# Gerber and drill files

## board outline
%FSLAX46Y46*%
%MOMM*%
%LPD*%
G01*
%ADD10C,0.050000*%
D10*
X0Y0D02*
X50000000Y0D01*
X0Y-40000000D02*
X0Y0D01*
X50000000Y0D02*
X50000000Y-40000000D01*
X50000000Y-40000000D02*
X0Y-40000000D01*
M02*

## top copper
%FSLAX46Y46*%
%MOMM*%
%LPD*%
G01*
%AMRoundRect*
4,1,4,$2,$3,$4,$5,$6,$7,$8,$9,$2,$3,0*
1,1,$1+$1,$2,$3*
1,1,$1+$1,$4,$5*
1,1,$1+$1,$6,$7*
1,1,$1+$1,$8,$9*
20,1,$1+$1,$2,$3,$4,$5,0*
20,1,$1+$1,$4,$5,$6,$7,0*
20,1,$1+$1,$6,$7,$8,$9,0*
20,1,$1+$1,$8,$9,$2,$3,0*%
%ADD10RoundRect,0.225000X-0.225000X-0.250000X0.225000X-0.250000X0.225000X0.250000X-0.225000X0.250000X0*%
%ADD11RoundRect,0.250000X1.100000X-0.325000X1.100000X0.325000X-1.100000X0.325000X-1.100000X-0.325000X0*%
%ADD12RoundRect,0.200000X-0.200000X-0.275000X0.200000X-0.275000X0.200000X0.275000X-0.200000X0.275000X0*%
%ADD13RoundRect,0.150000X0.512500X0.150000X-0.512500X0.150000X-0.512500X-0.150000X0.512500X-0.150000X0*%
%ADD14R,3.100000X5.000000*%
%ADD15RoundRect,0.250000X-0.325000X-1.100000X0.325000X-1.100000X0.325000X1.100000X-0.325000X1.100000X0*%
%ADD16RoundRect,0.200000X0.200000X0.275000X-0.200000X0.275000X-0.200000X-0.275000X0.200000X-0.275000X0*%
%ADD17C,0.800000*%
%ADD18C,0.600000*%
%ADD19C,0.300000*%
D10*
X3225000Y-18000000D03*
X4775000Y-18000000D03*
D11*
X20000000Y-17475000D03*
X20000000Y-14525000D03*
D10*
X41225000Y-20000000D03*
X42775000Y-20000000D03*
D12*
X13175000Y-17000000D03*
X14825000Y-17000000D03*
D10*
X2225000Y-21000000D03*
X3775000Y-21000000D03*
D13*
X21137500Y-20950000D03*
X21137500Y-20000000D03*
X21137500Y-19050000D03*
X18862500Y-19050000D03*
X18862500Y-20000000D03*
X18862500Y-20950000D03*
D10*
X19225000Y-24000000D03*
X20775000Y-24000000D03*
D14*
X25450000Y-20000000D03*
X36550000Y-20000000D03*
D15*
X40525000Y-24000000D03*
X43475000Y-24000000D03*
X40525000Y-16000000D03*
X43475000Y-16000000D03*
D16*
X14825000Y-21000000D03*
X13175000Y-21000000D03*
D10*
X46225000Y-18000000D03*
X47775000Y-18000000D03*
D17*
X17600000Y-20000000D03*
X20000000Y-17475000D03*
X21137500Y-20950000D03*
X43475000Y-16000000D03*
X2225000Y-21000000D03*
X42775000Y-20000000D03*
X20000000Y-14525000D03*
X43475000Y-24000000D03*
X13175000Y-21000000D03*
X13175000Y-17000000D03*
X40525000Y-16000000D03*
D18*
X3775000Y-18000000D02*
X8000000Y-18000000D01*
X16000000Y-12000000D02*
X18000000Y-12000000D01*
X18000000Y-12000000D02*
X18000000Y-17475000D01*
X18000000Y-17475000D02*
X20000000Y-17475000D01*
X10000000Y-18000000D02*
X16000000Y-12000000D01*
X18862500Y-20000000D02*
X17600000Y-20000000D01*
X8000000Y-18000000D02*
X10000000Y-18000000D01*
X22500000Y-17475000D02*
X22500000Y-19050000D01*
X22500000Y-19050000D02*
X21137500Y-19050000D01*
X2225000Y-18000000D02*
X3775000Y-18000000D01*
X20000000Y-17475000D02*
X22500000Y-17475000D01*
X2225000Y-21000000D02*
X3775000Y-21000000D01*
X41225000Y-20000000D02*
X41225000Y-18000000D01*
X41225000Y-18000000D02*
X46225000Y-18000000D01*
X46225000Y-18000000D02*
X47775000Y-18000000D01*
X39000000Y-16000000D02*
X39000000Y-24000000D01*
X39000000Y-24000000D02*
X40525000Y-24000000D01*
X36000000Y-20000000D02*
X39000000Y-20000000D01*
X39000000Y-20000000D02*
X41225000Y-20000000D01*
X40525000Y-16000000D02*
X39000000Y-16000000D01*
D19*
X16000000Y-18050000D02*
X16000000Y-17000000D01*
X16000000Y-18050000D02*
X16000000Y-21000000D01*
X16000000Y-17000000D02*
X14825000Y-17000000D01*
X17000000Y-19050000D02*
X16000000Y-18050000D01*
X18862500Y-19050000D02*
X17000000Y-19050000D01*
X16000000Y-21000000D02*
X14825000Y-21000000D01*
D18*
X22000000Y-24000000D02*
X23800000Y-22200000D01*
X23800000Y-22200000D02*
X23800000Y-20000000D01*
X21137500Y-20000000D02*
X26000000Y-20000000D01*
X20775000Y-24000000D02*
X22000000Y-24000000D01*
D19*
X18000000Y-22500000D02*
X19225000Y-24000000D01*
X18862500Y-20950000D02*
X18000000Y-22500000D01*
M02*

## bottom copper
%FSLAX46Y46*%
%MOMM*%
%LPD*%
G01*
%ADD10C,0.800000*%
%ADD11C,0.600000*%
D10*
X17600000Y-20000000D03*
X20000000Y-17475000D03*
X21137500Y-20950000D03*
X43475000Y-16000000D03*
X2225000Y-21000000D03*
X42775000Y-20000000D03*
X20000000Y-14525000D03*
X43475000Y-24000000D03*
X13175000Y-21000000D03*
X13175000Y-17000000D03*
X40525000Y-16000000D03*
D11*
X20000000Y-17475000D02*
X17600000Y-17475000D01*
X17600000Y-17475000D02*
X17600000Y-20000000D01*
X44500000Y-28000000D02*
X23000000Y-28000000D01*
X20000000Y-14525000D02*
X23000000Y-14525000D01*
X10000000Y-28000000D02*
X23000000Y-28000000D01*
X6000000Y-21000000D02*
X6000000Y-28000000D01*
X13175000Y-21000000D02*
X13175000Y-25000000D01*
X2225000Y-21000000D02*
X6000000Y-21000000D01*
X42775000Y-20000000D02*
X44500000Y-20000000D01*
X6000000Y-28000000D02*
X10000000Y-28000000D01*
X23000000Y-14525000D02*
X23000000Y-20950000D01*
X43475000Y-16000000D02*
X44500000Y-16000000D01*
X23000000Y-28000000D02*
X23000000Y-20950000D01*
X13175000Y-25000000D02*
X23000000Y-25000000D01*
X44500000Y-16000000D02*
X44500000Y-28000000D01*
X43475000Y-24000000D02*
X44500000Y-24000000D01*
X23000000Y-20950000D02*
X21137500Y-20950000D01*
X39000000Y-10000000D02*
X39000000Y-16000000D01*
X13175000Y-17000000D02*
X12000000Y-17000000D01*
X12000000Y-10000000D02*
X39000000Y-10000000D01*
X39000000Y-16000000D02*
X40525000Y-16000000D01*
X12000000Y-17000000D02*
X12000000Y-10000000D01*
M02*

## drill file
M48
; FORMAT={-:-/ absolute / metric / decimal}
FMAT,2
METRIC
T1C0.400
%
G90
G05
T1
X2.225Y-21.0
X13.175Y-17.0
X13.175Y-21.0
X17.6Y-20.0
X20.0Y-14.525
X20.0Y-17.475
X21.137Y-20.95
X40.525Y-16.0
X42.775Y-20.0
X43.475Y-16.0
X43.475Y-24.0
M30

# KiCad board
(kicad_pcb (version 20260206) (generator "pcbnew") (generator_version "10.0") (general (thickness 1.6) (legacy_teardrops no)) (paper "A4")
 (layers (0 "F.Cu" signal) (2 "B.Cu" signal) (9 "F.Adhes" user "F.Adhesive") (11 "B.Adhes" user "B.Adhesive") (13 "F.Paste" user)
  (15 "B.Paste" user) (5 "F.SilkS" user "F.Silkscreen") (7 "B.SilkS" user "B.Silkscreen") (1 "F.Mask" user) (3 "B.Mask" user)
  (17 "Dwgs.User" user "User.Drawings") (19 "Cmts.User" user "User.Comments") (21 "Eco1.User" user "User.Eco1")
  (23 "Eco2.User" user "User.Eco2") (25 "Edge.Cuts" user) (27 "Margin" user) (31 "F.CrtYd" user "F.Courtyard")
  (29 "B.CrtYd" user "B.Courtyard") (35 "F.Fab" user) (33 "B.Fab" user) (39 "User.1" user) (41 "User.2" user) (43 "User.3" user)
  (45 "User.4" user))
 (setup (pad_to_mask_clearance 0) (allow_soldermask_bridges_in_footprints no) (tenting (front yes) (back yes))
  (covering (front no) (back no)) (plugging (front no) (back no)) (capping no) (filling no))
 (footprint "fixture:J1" (layer "F.Cu") (at 4 18)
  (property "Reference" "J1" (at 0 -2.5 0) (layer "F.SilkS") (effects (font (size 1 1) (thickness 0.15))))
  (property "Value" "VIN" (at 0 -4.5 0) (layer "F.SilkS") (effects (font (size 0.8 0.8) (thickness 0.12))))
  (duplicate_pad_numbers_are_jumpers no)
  (pad "1" smd roundrect (at -0.775 0) (size 0.9 0.95) (layers "F.Cu" "F.Mask" "F.Paste") (roundrect_rratio 0.25) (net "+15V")
   (thermal_bridge_angle 45))
  (pad "2" smd roundrect (at 0.775 0) (size 0.9 0.95) (layers "F.Cu" "F.Mask" "F.Paste") (roundrect_rratio 0.25) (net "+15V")
   (thermal_bridge_angle 45)))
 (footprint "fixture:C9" (layer "F.Cu") (at 20 16 90)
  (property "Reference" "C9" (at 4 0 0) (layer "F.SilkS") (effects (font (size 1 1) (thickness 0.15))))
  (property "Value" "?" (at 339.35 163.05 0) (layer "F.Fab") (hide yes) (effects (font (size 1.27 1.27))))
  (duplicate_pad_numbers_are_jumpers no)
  (pad "1" smd roundrect (at -1.475 0 90) (size 1.15 2.7) (layers "F.Cu" "F.Mask" "F.Paste") (roundrect_rratio 0.217391) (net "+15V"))
  (pad "2" smd roundrect (at 1.475 0 90) (size 1.15 2.7) (layers "F.Cu" "F.Mask" "F.Paste") (roundrect_rratio 0.217391) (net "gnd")))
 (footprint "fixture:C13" (layer "F.Cu") (at 42 20)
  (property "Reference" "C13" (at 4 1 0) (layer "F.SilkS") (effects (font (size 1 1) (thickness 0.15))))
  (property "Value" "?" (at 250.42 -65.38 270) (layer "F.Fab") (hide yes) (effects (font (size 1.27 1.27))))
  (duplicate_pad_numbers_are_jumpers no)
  (pad "1" smd roundrect (at -0.775 0) (size 0.9 0.95) (layers "F.Cu" "F.Mask" "F.Paste") (roundrect_rratio 0.25) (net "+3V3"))
  (pad "2" smd roundrect (at 0.775 0) (size 0.9 0.95) (layers "F.Cu" "F.Mask" "F.Paste") (roundrect_rratio 0.25) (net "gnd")))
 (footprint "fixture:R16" (layer "F.Cu") (at 14 17)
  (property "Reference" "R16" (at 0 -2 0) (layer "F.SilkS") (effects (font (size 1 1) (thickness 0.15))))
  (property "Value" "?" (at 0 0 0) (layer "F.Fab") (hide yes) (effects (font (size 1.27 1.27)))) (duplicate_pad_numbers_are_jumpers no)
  (pad "1" smd roundrect (at -0.825 0) (size 0.8 0.95) (layers "F.Cu" "F.Mask" "F.Paste") (roundrect_rratio 0.25) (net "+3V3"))
  (pad "2" smd roundrect (at 0.825 0) (size 0.8 0.95) (layers "F.Cu" "F.Mask" "F.Paste") (roundrect_rratio 0.25) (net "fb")))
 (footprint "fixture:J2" (layer "F.Cu") (at 3 21)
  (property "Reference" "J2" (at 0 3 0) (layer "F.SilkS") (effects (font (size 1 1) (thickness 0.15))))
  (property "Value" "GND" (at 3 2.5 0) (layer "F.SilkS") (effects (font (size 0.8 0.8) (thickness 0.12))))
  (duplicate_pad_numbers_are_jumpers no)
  (pad "1" smd roundrect (at -0.775 0) (size 0.9 0.95) (layers "F.Cu" "F.Mask" "F.Paste") (roundrect_rratio 0.25) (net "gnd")
   (thermal_bridge_angle 45))
  (pad "2" smd roundrect (at 0.775 0) (size 0.9 0.95) (layers "F.Cu" "F.Mask" "F.Paste") (roundrect_rratio 0.25) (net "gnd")
   (thermal_bridge_angle 45)))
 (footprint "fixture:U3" (layer "F.Cu") (at 20 20 180)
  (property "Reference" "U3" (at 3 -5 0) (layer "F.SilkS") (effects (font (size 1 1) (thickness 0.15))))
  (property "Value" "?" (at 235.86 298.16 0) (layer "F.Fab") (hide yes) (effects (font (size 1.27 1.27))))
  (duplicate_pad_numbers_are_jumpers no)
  (pad "1" smd roundrect (at -1.1375 -0.95 180) (size 1.325 0.6) (layers "F.Cu" "F.Mask" "F.Paste") (roundrect_rratio 0.25) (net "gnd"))
  (pad "2" smd roundrect (at -1.1375 0 180) (size 1.325 0.6) (layers "F.Cu" "F.Mask" "F.Paste") (roundrect_rratio 0.25) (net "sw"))
  (pad "3" smd roundrect (at -1.1375 0.95 180) (size 1.325 0.6) (layers "F.Cu" "F.Mask" "F.Paste") (roundrect_rratio 0.25) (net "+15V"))
  (pad "4" smd roundrect (at 1.1375 0.95 180) (size 1.325 0.6) (layers "F.Cu" "F.Mask" "F.Paste") (roundrect_rratio 0.25) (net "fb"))
  (pad "5" smd roundrect (at 1.1375 0 180) (size 1.325 0.6) (layers "F.Cu" "F.Mask" "F.Paste") (roundrect_rratio 0.25) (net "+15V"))
  (pad "6" smd roundrect (at 1.1375 -0.95 180) (size 1.325 0.6) (layers "F.Cu" "F.Mask" "F.Paste") (roundrect_rratio 0.25) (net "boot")))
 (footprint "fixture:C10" (layer "F.Cu") (at 20 24)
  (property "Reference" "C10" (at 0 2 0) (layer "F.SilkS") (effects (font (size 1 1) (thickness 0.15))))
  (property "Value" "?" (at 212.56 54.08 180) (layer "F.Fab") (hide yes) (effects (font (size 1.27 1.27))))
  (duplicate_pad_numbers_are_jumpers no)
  (pad "1" smd roundrect (at -0.775 0) (size 0.9 0.95) (layers "F.Cu" "F.Mask" "F.Paste") (roundrect_rratio 0.25) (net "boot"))
  (pad "2" smd roundrect (at 0.775 0) (size 0.9 0.95) (layers "F.Cu" "F.Mask" "F.Paste") (roundrect_rratio 0.25) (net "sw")))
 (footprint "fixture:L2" (layer "F.Cu") (at 31 20)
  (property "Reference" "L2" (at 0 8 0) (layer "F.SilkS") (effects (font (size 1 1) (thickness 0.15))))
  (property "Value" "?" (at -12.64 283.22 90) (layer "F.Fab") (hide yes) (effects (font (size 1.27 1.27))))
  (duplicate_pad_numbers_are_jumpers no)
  (pad "1" smd rect (at -5.55 0) (size 3.1 5) (layers "F.Cu" "F.Mask" "F.Paste") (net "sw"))
  (pad "2" smd rect (at 5.55 0) (size 3.1 5) (layers "F.Cu" "F.Mask" "F.Paste") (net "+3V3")))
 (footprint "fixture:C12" (layer "F.Cu") (at 42 24)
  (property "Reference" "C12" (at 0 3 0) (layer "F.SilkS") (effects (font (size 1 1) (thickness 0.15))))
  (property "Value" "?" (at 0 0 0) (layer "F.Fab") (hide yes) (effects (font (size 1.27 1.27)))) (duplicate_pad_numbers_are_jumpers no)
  (pad "1" smd roundrect (at -1.475 0) (size 1.15 2.7) (layers "F.Cu" "F.Mask" "F.Paste") (roundrect_rratio 0.217391) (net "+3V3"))
  (pad "2" smd roundrect (at 1.475 0) (size 1.15 2.7) (layers "F.Cu" "F.Mask" "F.Paste") (roundrect_rratio 0.217391) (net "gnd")))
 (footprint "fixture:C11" (layer "F.Cu") (at 42 16)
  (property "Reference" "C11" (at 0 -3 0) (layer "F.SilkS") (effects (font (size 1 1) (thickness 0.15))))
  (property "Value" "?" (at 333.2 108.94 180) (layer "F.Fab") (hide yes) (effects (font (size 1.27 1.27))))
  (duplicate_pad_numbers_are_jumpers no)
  (pad "1" smd roundrect (at -1.475 0) (size 1.15 2.7) (layers "F.Cu" "F.Mask" "F.Paste") (roundrect_rratio 0.217391) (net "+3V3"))
  (pad "2" smd roundrect (at 1.475 0) (size 1.15 2.7) (layers "F.Cu" "F.Mask" "F.Paste") (roundrect_rratio 0.217391) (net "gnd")))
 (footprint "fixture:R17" (layer "F.Cu") (at 14 21 180)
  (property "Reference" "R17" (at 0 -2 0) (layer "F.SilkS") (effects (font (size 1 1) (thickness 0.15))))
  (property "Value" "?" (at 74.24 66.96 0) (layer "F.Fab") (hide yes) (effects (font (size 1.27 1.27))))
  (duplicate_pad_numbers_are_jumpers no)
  (pad "1" smd roundrect (at -0.825 0 180) (size 0.8 0.95) (layers "F.Cu" "F.Mask" "F.Paste") (roundrect_rratio 0.25) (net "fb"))
  (pad "2" smd roundrect (at 0.825 0 180) (size 0.8 0.95) (layers "F.Cu" "F.Mask" "F.Paste") (roundrect_rratio 0.25) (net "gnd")))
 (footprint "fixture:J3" (layer "F.Cu") (at 47 18)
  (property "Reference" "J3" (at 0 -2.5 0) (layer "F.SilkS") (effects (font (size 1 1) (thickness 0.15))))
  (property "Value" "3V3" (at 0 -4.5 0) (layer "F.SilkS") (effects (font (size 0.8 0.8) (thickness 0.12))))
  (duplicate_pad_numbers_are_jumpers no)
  (pad "1" smd roundrect (at -0.775 0) (size 0.9 0.95) (layers "F.Cu" "F.Mask" "F.Paste") (roundrect_rratio 0.25) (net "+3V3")
   (thermal_bridge_angle 45))
  (pad "2" smd roundrect (at 0.775 0) (size 0.9 0.95) (layers "F.Cu" "F.Mask" "F.Paste") (roundrect_rratio 0.25) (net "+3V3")
   (thermal_bridge_angle 45)))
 (gr_line (start 0 0) (end 50 0) (stroke (width 0.05) (type default)) (layer "Edge.Cuts"))
 (gr_line (start 0 40) (end 0 0) (stroke (width 0.05) (type default)) (layer "Edge.Cuts"))
 (gr_line (start 50 0) (end 50 40) (stroke (width 0.05) (type default)) (layer "Edge.Cuts"))
 (gr_line (start 50 40) (end 0 40) (stroke (width 0.05) (type default)) (layer "Edge.Cuts"))
 (segment (start 3.775 18) (end 8 18) (width 0.6) (layer "F.Cu") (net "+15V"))
 (segment (start 16 12) (end 18 12) (width 0.6) (layer "F.Cu") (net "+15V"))
 (segment (start 18 12) (end 18 17.475) (width 0.6) (layer "F.Cu") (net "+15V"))
 (segment (start 18 17.475) (end 20 17.475) (width 0.6) (layer "F.Cu") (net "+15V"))
 (segment (start 10 18) (end 16 12) (width 0.6) (layer "F.Cu") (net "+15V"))
 (segment (start 18.8625 20) (end 17.6 20) (width 0.6) (layer "F.Cu") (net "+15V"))
 (segment (start 8 18) (end 10 18) (width 0.6) (layer "F.Cu") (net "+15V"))
 (segment (start 22.5 17.475) (end 22.5 19.05) (width 0.6) (layer "F.Cu") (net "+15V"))
 (segment (start 22.5 19.05) (end 21.1375 19.05) (width 0.6) (layer "F.Cu") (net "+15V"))
 (segment (start 2.225 18) (end 3.775 18) (width 0.6) (layer "F.Cu") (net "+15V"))
 (segment (start 20 17.475) (end 22.5 17.475) (width 0.6) (layer "F.Cu") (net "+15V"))
 (via (at 17.6 20) (size 0.8) (drill 0.4) (layers "F.Cu" "B.Cu") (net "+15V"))
 (via (at 20 17.475) (size 0.8) (drill 0.4) (layers "F.Cu" "B.Cu") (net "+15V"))
 (segment (start 20 17.475) (end 17.6 17.475) (width 0.6) (layer "B.Cu") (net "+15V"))
 (segment (start 17.6 17.475) (end 17.6 20) (width 0.6) (layer "B.Cu") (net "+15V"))
 (segment (start 2.225 21) (end 3.775 21) (width 0.6) (layer "F.Cu") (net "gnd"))
 (via (at 21.1375 20.95) (size 0.8) (drill 0.4) (layers "F.Cu" "B.Cu") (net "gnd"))
 (via (at 43.475 16) (size 0.8) (drill 0.4) (layers "F.Cu" "B.Cu") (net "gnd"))
 (via (at 2.225 21) (size 0.8) (drill 0.4) (layers "F.Cu" "B.Cu") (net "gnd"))
 (via (at 42.775 20) (size 0.8) (drill 0.4) (layers "F.Cu" "B.Cu") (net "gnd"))
 (via (at 20 14.525) (size 0.8) (drill 0.4) (layers "F.Cu" "B.Cu") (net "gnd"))
 (via (at 43.475 24) (size 0.8) (drill 0.4) (layers "F.Cu" "B.Cu") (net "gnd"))
 (via (at 13.175 21) (size 0.8) (drill 0.4) (layers "F.Cu" "B.Cu") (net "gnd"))
 (segment (start 44.5 28) (end 23 28) (width 0.6) (layer "B.Cu") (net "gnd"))
 (segment (start 20 14.525) (end 23 14.525) (width 0.6) (layer "B.Cu") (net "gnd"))
 (segment (start 10 28) (end 23 28) (width 0.6) (layer "B.Cu") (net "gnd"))
 (segment (start 6 21) (end 6 28) (width 0.6) (layer "B.Cu") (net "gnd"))
 (segment (start 13.175 21) (end 13.175 25) (width 0.6) (layer "B.Cu") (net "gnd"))
 (segment (start 2.225 21) (end 6 21) (width 0.6) (layer "B.Cu") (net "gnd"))
 (segment (start 42.775 20) (end 44.5 20) (width 0.6) (layer "B.Cu") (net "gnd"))
 (segment (start 6 28) (end 10 28) (width 0.6) (layer "B.Cu") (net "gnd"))
 (segment (start 23 14.525) (end 23 20.95) (width 0.6) (layer "B.Cu") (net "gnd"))
 (segment (start 43.475 16) (end 44.5 16) (width 0.6) (layer "B.Cu") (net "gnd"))
 (segment (start 23 28) (end 23 20.95) (width 0.6) (layer "B.Cu") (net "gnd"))
 (segment (start 13.175 25) (end 23 25) (width 0.6) (layer "B.Cu") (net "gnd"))
 (segment (start 44.5 16) (end 44.5 28) (width 0.6) (layer "B.Cu") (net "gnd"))
 (segment (start 43.475 24) (end 44.5 24) (width 0.6) (layer "B.Cu") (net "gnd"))
 (segment (start 23 20.95) (end 21.1375 20.95) (width 0.6) (layer "B.Cu") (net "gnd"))
 (segment (start 41.225 20) (end 41.225 18) (width 0.6) (layer "F.Cu") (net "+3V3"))
 (segment (start 41.225 18) (end 46.225 18) (width 0.6) (layer "F.Cu") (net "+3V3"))
 (segment (start 46.225 18) (end 47.775 18) (width 0.6) (layer "F.Cu") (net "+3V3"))
 (segment (start 39 16) (end 39 24) (width 0.6) (layer "F.Cu") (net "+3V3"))
 (segment (start 39 24) (end 40.525 24) (width 0.6) (layer "F.Cu") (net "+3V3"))
 (segment (start 36 20) (end 39 20) (width 0.6) (layer "F.Cu") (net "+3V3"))
 (segment (start 39 20) (end 41.225 20) (width 0.6) (layer "F.Cu") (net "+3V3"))
 (segment (start 40.525 16) (end 39 16) (width 0.6) (layer "F.Cu") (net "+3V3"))
 (via (at 13.175 17) (size 0.8) (drill 0.4) (layers "F.Cu" "B.Cu") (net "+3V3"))
 (via (at 40.525 16) (size 0.8) (drill 0.4) (layers "F.Cu" "B.Cu") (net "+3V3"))
 (segment (start 39 10) (end 39 16) (width 0.6) (layer "B.Cu") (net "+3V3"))
 (segment (start 13.175 17) (end 12 17) (width 0.6) (layer "B.Cu") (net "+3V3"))
 (segment (start 12 10) (end 39 10) (width 0.6) (layer "B.Cu") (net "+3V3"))
 (segment (start 39 16) (end 40.525 16) (width 0.6) (layer "B.Cu") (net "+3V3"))
 (segment (start 12 17) (end 12 10) (width 0.6) (layer "B.Cu") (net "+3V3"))
 (segment (start 16 18.05) (end 16 17) (width 0.3) (layer "F.Cu") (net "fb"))
 (segment (start 16 18.05) (end 16 21) (width 0.3) (layer "F.Cu") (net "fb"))
 (segment (start 16 17) (end 14.825 17) (width 0.3) (layer "F.Cu") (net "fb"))
 (segment (start 17 19.05) (end 16 18.05) (width 0.3) (layer "F.Cu") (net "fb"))
 (segment (start 18.8625 19.05) (end 17 19.05) (width 0.3) (layer "F.Cu") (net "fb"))
 (segment (start 16 21) (end 14.825 21) (width 0.3) (layer "F.Cu") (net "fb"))
 (segment (start 22 24) (end 23.8 22.2) (width 0.6) (layer "F.Cu") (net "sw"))
 (segment (start 23.8 22.2) (end 23.8 20) (width 0.6) (layer "F.Cu") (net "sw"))
 (segment (start 21.1375 20) (end 26 20) (width 0.6) (layer "F.Cu") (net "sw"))
 (segment (start 20.775 24) (end 22 24) (width 0.6) (layer "F.Cu") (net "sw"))
 (segment (start 18 22.5) (end 19.225 24) (width 0.3) (layer "F.Cu") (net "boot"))
 (segment (start 18.8625 20.95) (end 18 22.5) (width 0.3) (layer "F.Cu") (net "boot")))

